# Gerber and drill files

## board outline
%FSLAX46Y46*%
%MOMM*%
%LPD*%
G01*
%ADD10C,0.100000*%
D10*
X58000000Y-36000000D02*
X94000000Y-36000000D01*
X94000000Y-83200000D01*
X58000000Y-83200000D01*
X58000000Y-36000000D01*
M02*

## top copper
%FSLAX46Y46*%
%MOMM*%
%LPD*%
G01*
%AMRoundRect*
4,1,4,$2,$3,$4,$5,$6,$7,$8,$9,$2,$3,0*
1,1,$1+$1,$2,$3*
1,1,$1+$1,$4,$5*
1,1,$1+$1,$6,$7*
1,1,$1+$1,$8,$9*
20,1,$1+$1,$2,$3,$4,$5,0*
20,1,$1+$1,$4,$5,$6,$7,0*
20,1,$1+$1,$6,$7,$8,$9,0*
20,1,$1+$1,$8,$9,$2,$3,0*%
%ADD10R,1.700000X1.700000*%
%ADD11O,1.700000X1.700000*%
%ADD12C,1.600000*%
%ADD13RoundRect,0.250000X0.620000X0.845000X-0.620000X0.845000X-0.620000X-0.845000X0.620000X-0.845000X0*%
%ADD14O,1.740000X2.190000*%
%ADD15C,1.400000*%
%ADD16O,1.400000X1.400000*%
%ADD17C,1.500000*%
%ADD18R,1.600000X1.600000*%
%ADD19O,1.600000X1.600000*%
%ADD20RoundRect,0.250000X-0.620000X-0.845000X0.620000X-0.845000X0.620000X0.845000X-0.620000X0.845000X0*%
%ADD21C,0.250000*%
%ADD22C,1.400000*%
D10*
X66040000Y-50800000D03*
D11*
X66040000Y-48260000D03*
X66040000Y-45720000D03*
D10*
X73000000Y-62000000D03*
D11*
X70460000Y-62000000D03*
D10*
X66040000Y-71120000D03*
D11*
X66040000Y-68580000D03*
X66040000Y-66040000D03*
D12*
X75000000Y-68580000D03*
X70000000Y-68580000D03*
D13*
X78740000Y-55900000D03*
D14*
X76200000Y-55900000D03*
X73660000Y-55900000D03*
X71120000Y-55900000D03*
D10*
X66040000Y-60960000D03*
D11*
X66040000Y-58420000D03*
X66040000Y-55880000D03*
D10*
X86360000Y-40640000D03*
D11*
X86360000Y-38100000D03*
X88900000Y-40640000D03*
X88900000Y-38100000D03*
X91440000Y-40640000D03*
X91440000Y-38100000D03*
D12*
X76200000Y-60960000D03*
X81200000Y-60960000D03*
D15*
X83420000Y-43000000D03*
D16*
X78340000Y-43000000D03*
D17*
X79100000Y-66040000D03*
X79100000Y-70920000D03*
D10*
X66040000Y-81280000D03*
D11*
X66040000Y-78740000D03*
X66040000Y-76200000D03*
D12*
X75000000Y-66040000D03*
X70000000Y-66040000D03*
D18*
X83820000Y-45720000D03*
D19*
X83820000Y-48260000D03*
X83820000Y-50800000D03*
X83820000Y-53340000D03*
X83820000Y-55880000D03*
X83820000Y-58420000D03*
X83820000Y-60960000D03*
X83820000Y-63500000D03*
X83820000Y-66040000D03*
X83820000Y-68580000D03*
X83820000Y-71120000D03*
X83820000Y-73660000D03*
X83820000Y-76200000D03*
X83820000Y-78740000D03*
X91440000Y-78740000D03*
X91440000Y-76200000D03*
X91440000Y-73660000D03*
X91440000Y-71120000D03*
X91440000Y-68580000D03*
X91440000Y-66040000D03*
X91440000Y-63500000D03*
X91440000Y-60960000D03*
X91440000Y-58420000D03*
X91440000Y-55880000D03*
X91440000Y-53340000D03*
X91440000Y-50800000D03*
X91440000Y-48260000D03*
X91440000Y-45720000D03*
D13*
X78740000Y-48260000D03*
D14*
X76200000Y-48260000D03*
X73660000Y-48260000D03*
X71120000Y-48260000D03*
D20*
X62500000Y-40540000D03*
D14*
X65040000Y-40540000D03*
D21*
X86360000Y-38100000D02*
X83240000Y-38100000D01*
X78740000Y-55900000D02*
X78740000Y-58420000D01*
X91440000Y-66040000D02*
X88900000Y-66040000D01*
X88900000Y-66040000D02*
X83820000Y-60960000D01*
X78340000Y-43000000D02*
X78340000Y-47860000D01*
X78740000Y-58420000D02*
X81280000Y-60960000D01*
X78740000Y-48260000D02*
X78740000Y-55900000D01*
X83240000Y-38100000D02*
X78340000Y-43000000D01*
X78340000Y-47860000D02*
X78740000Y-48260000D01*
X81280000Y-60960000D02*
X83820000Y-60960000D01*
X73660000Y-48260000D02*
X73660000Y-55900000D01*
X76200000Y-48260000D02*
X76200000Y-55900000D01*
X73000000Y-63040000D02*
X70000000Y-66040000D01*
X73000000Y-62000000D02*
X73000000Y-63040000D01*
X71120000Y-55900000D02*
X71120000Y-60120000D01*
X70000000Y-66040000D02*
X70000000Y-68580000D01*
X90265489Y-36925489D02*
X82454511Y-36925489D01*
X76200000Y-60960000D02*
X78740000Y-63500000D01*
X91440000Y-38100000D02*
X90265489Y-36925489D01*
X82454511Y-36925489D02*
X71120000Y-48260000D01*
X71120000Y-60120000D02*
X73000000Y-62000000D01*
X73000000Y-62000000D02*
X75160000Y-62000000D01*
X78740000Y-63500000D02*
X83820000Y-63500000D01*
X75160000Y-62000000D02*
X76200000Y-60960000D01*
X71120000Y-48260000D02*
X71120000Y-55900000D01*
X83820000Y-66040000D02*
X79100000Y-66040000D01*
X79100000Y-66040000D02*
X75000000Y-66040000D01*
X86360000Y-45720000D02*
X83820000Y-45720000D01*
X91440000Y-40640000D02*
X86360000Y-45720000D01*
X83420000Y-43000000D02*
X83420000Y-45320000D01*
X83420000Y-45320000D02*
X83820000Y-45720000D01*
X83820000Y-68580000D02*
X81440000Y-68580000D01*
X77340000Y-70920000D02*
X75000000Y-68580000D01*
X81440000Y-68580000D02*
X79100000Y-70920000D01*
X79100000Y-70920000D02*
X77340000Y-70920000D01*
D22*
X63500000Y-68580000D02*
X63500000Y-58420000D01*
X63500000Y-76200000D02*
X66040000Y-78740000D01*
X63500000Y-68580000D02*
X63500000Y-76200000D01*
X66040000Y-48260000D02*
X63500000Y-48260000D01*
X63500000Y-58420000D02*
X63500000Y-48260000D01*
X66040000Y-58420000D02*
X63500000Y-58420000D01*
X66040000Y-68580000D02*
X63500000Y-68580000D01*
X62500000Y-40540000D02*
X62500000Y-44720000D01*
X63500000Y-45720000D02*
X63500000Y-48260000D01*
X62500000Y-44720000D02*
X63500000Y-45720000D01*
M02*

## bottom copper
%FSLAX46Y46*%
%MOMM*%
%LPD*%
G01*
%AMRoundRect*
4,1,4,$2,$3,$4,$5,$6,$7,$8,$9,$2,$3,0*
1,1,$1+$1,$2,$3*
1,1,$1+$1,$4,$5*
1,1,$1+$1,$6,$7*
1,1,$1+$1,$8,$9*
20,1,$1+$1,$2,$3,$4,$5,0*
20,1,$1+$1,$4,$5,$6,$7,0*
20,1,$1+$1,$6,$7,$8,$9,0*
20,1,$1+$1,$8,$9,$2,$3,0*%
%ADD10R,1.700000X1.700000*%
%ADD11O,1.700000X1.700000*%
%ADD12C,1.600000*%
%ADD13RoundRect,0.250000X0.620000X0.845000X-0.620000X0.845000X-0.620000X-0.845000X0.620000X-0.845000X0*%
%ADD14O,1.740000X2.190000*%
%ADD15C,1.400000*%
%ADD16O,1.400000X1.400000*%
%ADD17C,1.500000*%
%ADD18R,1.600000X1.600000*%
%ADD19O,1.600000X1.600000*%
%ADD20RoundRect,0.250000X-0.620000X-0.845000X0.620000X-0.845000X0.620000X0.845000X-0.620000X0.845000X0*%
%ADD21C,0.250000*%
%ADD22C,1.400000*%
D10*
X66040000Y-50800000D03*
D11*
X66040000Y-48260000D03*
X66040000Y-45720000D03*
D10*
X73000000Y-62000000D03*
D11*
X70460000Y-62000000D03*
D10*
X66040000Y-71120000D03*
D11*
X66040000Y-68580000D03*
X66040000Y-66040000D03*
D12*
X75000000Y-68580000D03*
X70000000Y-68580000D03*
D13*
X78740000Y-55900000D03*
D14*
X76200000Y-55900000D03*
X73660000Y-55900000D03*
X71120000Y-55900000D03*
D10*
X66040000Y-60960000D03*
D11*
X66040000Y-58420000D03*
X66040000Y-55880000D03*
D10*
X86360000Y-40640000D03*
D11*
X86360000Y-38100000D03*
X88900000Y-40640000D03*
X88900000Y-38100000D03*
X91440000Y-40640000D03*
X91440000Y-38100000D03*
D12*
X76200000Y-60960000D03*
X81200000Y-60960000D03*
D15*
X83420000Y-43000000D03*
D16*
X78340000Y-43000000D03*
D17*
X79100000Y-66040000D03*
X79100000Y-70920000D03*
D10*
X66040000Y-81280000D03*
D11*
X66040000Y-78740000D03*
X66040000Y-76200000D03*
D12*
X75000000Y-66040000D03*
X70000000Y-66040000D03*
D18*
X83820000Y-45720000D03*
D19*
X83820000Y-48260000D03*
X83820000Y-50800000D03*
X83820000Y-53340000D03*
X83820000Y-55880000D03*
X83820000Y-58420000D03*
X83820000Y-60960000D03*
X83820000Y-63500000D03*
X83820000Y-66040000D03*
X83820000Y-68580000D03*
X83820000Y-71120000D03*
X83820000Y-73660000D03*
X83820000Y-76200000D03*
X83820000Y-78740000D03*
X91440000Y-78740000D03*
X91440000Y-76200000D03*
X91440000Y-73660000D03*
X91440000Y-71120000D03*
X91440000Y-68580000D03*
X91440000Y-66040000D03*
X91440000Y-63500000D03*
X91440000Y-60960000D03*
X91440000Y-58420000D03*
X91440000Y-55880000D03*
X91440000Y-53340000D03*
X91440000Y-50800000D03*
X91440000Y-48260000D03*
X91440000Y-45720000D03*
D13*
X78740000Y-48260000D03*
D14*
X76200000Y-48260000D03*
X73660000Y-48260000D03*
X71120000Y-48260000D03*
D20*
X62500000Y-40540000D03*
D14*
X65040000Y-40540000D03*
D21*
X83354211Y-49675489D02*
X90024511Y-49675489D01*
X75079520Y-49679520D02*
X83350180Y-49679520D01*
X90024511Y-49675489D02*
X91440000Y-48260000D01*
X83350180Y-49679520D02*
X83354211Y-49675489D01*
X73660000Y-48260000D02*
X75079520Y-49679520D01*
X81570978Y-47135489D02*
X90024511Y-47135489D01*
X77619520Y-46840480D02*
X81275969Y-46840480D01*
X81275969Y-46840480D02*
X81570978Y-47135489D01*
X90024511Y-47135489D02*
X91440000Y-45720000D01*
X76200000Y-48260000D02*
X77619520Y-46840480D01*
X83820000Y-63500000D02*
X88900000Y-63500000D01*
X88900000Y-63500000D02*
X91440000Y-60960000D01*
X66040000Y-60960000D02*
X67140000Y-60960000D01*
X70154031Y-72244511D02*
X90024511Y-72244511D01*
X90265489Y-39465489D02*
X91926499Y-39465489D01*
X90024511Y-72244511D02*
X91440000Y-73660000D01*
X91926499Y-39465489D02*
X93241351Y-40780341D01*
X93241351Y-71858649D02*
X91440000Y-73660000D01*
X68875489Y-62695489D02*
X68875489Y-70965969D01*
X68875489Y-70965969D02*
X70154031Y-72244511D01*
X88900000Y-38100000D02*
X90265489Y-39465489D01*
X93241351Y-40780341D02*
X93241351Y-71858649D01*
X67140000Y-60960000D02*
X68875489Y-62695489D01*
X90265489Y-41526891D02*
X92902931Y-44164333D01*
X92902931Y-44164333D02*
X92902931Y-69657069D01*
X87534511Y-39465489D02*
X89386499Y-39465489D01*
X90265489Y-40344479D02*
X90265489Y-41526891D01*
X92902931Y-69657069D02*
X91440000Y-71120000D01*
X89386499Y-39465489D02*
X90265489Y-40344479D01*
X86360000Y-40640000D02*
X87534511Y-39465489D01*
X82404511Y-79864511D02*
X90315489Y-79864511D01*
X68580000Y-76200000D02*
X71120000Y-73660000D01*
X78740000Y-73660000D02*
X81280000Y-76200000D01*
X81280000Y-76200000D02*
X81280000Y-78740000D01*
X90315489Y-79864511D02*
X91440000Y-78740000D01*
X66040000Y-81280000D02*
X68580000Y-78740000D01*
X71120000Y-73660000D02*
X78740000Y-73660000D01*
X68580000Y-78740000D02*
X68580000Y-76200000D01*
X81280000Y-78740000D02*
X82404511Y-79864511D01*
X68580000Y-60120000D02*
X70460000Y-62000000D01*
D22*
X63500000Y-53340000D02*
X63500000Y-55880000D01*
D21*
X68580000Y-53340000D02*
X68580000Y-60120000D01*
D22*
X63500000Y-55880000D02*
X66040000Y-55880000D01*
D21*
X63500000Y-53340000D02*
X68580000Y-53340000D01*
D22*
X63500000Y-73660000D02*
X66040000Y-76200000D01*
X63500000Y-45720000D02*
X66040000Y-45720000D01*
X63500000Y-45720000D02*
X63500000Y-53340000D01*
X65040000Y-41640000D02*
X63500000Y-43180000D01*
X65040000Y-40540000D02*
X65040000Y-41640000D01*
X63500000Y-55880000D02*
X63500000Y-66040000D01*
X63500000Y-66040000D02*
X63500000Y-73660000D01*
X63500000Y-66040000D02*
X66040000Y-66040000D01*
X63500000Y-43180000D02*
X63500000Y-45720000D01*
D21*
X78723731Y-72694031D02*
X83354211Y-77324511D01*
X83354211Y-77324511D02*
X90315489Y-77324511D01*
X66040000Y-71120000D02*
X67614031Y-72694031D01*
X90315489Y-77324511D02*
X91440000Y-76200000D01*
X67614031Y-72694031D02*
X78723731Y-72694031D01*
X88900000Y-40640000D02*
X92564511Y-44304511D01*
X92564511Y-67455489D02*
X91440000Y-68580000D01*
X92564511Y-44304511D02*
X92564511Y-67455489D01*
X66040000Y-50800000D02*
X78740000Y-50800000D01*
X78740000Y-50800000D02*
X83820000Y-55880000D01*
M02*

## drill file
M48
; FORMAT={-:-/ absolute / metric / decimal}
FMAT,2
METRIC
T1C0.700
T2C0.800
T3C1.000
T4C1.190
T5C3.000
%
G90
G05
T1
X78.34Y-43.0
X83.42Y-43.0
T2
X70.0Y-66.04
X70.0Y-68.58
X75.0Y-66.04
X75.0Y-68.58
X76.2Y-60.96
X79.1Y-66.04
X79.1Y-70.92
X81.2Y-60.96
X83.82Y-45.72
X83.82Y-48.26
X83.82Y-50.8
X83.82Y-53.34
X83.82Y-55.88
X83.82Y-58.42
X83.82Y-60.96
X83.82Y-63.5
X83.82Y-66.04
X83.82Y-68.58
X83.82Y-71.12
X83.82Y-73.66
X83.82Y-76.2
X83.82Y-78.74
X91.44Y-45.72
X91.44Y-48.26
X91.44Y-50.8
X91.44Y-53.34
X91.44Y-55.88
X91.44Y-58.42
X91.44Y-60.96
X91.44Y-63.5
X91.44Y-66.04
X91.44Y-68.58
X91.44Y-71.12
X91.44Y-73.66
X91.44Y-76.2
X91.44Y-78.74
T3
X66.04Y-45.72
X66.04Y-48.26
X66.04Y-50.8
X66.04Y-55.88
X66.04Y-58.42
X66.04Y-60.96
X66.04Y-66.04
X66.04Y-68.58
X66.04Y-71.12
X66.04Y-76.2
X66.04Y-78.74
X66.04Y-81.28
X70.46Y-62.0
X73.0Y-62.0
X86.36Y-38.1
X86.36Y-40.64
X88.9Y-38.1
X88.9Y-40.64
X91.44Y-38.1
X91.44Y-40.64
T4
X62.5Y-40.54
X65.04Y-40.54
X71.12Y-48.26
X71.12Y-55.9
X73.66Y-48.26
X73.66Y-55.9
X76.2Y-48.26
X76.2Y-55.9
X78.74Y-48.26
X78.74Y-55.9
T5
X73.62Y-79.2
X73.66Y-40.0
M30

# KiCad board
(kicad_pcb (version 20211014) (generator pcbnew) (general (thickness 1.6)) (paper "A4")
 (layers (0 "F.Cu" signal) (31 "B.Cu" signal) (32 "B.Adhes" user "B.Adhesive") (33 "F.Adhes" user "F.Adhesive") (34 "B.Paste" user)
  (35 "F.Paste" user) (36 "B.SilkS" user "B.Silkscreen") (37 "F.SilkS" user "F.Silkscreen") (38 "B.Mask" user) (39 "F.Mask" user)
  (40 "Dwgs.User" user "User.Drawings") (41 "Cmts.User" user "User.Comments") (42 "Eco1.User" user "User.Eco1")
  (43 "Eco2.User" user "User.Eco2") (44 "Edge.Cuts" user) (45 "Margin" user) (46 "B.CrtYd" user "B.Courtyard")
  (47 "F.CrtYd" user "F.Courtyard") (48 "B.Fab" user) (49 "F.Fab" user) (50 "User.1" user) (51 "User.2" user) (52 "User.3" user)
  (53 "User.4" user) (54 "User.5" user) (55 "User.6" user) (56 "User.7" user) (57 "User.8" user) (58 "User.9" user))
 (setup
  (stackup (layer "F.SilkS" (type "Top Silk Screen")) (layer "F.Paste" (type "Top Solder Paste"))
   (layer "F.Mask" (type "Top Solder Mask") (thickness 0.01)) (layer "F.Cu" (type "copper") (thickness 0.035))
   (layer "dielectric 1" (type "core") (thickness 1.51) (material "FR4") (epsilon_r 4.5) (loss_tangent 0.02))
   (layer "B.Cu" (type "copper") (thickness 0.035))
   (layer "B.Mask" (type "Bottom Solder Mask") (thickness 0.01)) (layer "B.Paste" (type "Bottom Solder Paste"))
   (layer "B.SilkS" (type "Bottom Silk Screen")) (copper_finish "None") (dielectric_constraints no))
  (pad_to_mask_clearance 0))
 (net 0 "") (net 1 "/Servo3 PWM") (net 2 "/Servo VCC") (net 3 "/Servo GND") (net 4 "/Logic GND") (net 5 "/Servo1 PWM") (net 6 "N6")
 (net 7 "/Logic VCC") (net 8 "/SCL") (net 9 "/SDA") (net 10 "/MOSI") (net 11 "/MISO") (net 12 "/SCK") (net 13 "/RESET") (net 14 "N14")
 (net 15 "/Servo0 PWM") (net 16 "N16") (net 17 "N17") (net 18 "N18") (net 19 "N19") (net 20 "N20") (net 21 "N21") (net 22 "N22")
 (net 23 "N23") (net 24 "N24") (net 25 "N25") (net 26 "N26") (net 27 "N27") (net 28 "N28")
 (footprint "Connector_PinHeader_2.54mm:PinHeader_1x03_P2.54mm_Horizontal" (layer "F.Cu") (at 66.04 50.8 180)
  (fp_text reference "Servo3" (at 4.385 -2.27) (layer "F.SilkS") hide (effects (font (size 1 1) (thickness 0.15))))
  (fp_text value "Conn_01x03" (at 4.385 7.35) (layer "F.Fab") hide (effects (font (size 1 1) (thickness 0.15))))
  (pad "1" thru_hole rect (at 0 0 180) (size 1.7 1.7) (drill 1) (layers *.Cu *.Mask) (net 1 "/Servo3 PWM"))
  (pad "2" thru_hole oval (at 0 2.54 180) (size 1.7 1.7) (drill 1) (layers *.Cu *.Mask) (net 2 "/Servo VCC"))
  (pad "3" thru_hole oval (at 0 5.08 180) (size 1.7 1.7) (drill 1) (layers *.Cu *.Mask) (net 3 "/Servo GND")))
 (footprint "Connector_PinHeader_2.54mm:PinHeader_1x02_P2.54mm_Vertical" (layer "F.Cu") (at 73 62 -90)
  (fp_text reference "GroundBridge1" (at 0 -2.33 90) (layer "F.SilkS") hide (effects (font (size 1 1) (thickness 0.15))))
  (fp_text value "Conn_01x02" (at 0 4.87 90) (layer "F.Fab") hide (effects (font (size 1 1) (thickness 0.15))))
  (pad "1" thru_hole rect (at 0 0 270) (size 1.7 1.7) (drill 1) (layers *.Cu *.Mask) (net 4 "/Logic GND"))
  (pad "2" thru_hole oval (at 0 2.54 270) (size 1.7 1.7) (drill 1) (layers *.Cu *.Mask) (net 3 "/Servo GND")))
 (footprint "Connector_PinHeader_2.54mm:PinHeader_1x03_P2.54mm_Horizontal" (layer "F.Cu") (at 66.04 71.12 180)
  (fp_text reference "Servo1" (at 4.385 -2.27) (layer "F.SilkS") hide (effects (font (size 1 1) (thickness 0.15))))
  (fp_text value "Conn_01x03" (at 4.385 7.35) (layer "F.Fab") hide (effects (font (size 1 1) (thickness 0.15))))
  (pad "1" thru_hole rect (at 0 0 180) (size 1.7 1.7) (drill 1) (layers *.Cu *.Mask) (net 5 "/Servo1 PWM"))
  (pad "2" thru_hole oval (at 0 2.54 180) (size 1.7 1.7) (drill 1) (layers *.Cu *.Mask) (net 2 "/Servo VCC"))
  (pad "3" thru_hole oval (at 0 5.08 180) (size 1.7 1.7) (drill 1) (layers *.Cu *.Mask) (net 3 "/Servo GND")))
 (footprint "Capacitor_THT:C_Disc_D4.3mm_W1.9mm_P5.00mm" (layer "F.Cu") (at 75 68.58 180)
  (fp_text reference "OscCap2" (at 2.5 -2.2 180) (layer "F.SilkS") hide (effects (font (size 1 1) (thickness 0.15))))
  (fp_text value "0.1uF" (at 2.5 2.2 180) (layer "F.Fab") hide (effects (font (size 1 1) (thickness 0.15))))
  (pad "1" thru_hole circle (at 0 0 180) (size 1.6 1.6) (drill 0.8) (layers *.Cu *.Mask) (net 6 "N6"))
  (pad "2" thru_hole circle (at 5 0 180) (size 1.6 1.6) (drill 0.8) (layers *.Cu *.Mask) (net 4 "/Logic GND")))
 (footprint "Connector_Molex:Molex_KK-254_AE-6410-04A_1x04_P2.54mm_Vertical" (layer "F.Cu") (at 78.74 55.9 180)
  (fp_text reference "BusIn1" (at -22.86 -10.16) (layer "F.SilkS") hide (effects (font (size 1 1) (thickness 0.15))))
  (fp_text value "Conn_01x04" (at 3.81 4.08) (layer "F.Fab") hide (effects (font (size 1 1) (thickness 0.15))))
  (pad "1" thru_hole roundrect (at 0 0 180) (size 1.74 2.19) (drill 1.19) (layers *.Cu *.Mask) (roundrect_rratio 0.1436781609)
   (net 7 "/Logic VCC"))
  (pad "2" thru_hole oval (at 2.54 0 180) (size 1.74 2.19) (drill 1.19) (layers *.Cu *.Mask) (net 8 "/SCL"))
  (pad "3" thru_hole oval (at 5.08 0 180) (size 1.74 2.19) (drill 1.19) (layers *.Cu *.Mask) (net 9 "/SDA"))
  (pad "4" thru_hole oval (at 7.62 0 180) (size 1.74 2.19) (drill 1.19) (layers *.Cu *.Mask) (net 4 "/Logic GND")))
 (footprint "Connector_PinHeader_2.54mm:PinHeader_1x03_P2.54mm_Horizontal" (layer "F.Cu") (at 66.04 60.96 180)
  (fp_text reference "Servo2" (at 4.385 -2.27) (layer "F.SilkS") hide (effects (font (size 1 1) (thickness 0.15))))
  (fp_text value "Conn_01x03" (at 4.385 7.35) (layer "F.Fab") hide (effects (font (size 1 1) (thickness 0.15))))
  (pad "1" thru_hole rect (at 0 0 180) (size 1.7 1.7) (drill 1) (layers *.Cu *.Mask) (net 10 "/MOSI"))
  (pad "2" thru_hole oval (at 0 2.54 180) (size 1.7 1.7) (drill 1) (layers *.Cu *.Mask) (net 2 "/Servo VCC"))
  (pad "3" thru_hole oval (at 0 5.08 180) (size 1.7 1.7) (drill 1) (layers *.Cu *.Mask) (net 3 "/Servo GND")))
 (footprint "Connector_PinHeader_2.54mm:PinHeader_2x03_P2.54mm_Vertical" (layer "F.Cu") (at 86.36 40.64 90)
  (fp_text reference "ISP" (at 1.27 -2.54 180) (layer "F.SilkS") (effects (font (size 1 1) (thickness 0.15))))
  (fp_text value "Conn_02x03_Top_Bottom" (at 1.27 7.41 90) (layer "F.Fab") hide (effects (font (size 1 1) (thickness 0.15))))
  (pad "1" thru_hole rect (at 0 0 90) (size 1.7 1.7) (drill 1) (layers *.Cu *.Mask) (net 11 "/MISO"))
  (pad "2" thru_hole oval (at 2.54 0 90) (size 1.7 1.7) (drill 1) (layers *.Cu *.Mask) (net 7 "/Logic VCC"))
  (pad "3" thru_hole oval (at 0 2.54 90) (size 1.7 1.7) (drill 1) (layers *.Cu *.Mask) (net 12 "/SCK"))
  (pad "4" thru_hole oval (at 2.54 2.54 90) (size 1.7 1.7) (drill 1) (layers *.Cu *.Mask) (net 10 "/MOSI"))
  (pad "5" thru_hole oval (at 0 5.08 90) (size 1.7 1.7) (drill 1) (layers *.Cu *.Mask) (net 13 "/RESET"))
  (pad "6" thru_hole oval (at 2.54 5.08 90) (size 1.7 1.7) (drill 1) (layers *.Cu *.Mask) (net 4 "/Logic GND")))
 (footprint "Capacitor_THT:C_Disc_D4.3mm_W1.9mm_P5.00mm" (layer "F.Cu") (at 76.2 60.96)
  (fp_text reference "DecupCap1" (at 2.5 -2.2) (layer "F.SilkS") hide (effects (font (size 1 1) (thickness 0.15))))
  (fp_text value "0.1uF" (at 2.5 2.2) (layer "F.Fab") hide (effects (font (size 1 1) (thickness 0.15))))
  (pad "1" thru_hole circle (at 0 0) (size 1.6 1.6) (drill 0.8) (layers *.Cu *.Mask) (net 4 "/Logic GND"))
  (pad "2" thru_hole circle (at 5 0) (size 1.6 1.6) (drill 0.8) (layers *.Cu *.Mask) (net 7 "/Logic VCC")))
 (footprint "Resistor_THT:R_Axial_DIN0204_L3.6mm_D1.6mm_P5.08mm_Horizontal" (layer "F.Cu") (at 83.42 43 180)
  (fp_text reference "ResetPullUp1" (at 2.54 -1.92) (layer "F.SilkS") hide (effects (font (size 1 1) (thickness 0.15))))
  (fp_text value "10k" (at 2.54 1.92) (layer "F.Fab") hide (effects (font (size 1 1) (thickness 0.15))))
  (pad "1" thru_hole circle (at 0 0 180) (size 1.4 1.4) (drill 0.7) (layers *.Cu *.Mask) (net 13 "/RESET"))
  (pad "2" thru_hole oval (at 5.08 0 180) (size 1.4 1.4) (drill 0.7) (layers *.Cu *.Mask) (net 7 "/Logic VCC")))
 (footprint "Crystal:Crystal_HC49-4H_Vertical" (layer "F.Cu") (at 79.1 66.04 -90)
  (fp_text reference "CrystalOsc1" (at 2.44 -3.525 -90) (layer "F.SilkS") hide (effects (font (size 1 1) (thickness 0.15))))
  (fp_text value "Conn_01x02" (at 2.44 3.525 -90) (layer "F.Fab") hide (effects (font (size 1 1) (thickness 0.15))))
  (pad "1" thru_hole circle (at 0 0 270) (size 1.5 1.5) (drill 0.8) (layers *.Cu *.Mask) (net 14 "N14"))
  (pad "2" thru_hole circle (at 4.88 0 270) (size 1.5 1.5) (drill 0.8) (layers *.Cu *.Mask) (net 6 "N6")))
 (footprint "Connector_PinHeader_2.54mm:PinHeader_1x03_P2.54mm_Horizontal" (layer "F.Cu") (at 66.04 81.28 180)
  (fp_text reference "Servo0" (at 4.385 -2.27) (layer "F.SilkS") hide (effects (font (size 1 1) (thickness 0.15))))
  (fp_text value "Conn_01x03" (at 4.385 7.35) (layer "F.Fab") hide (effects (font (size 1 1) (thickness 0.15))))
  (pad "1" thru_hole rect (at 0 0 180) (size 1.7 1.7) (drill 1) (layers *.Cu *.Mask) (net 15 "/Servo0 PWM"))
  (pad "2" thru_hole oval (at 0 2.54 180) (size 1.7 1.7) (drill 1) (layers *.Cu *.Mask) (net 2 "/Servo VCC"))
  (pad "3" thru_hole oval (at 0 5.08 180) (size 1.7 1.7) (drill 1) (layers *.Cu *.Mask) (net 3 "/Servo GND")))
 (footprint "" (layer "F.Cu") (at 73.66 40)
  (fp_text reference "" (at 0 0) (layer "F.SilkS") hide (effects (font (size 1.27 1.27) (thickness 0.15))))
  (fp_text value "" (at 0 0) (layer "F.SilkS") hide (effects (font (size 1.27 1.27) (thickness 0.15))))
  (pad "" np_thru_hole circle (at 0 0) (size 6 6) (drill 3) (layers *.Mask)))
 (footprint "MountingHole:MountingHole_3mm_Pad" (layer "F.Cu") (at 73.62 79.2)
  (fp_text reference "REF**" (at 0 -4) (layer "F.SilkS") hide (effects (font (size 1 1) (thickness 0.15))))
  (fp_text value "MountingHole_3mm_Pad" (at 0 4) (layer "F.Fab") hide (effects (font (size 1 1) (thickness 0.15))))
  (pad "" np_thru_hole circle (at 0 0) (size 6 6) (drill 3) (layers *.Mask)))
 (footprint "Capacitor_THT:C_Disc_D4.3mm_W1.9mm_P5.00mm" (layer "F.Cu") (at 75 66.04 180)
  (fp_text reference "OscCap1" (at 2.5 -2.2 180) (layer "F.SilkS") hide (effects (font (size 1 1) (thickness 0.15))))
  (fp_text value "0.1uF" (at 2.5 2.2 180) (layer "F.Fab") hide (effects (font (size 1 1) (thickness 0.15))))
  (pad "1" thru_hole circle (at 0 0 180) (size 1.6 1.6) (drill 0.8) (layers *.Cu *.Mask) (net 14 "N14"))
  (pad "2" thru_hole circle (at 5 0 180) (size 1.6 1.6) (drill 0.8) (layers *.Cu *.Mask) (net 4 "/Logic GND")))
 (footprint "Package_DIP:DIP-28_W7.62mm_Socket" (layer "F.Cu") (at 83.82 45.72)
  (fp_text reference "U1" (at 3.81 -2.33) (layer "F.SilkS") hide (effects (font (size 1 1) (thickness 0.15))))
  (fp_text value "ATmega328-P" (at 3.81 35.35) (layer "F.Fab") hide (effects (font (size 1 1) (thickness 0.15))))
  (pad "1" thru_hole rect (at 0 0) (size 1.6 1.6) (drill 0.8) (layers *.Cu *.Mask) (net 13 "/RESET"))
  (pad "2" thru_hole oval (at 0 2.54) (size 1.6 1.6) (drill 0.8) (layers *.Cu *.Mask) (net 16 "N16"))
  (pad "3" thru_hole oval (at 0 5.08) (size 1.6 1.6) (drill 0.8) (layers *.Cu *.Mask) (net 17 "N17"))
  (pad "4" thru_hole oval (at 0 7.62) (size 1.6 1.6) (drill 0.8) (layers *.Cu *.Mask) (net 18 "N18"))
  (pad "5" thru_hole oval (at 0 10.16) (size 1.6 1.6) (drill 0.8) (layers *.Cu *.Mask) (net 1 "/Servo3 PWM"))
  (pad "6" thru_hole oval (at 0 12.7) (size 1.6 1.6) (drill 0.8) (layers *.Cu *.Mask) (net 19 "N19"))
  (pad "7" thru_hole oval (at 0 15.24) (size 1.6 1.6) (drill 0.8) (layers *.Cu *.Mask) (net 7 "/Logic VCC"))
  (pad "8" thru_hole oval (at 0 17.78) (size 1.6 1.6) (drill 0.8) (layers *.Cu *.Mask) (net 4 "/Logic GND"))
  (pad "9" thru_hole oval (at 0 20.32) (size 1.6 1.6) (drill 0.8) (layers *.Cu *.Mask) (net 14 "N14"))
  (pad "10" thru_hole oval (at 0 22.86) (size 1.6 1.6) (drill 0.8) (layers *.Cu *.Mask) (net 6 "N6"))
  (pad "11" thru_hole oval (at 0 25.4) (size 1.6 1.6) (drill 0.8) (layers *.Cu *.Mask) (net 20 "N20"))
  (pad "12" thru_hole oval (at 0 27.94) (size 1.6 1.6) (drill 0.8) (layers *.Cu *.Mask) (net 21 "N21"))
  (pad "13" thru_hole oval (at 0 30.48) (size 1.6 1.6) (drill 0.8) (layers *.Cu *.Mask) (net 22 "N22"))
  (pad "14" thru_hole oval (at 0 33.02) (size 1.6 1.6) (drill 0.8) (layers *.Cu *.Mask) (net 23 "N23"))
  (pad "15" thru_hole oval (at 7.62 33.02) (size 1.6 1.6) (drill 0.8) (layers *.Cu *.Mask) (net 15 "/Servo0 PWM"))
  (pad "16" thru_hole oval (at 7.62 30.48) (size 1.6 1.6) (drill 0.8) (layers *.Cu *.Mask) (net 5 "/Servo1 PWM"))
  (pad "17" thru_hole oval (at 7.62 27.94) (size 1.6 1.6) (drill 0.8) (layers *.Cu *.Mask) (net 10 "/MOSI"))
  (pad "18" thru_hole oval (at 7.62 25.4) (size 1.6 1.6) (drill 0.8) (layers *.Cu *.Mask) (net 11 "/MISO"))
  (pad "19" thru_hole oval (at 7.62 22.86) (size 1.6 1.6) (drill 0.8) (layers *.Cu *.Mask) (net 12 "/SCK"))
  (pad "20" thru_hole oval (at 7.62 20.32) (size 1.6 1.6) (drill 0.8) (layers *.Cu *.Mask) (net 7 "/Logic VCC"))
  (pad "21" thru_hole oval (at 7.62 17.78) (size 1.6 1.6) (drill 0.8) (layers *.Cu *.Mask) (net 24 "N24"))
  (pad "22" thru_hole oval (at 7.62 15.24) (size 1.6 1.6) (drill 0.8) (layers *.Cu *.Mask) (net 4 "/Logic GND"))
  (pad "23" thru_hole oval (at 7.62 12.7) (size 1.6 1.6) (drill 0.8) (layers *.Cu *.Mask) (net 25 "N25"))
  (pad "24" thru_hole oval (at 7.62 10.16) (size 1.6 1.6) (drill 0.8) (layers *.Cu *.Mask) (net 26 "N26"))
  (pad "25" thru_hole oval (at 7.62 7.62) (size 1.6 1.6) (drill 0.8) (layers *.Cu *.Mask) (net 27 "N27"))
  (pad "26" thru_hole oval (at 7.62 5.08) (size 1.6 1.6) (drill 0.8) (layers *.Cu *.Mask) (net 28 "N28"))
  (pad "27" thru_hole oval (at 7.62 2.54) (size 1.6 1.6) (drill 0.8) (layers *.Cu *.Mask) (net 9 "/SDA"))
  (pad "28" thru_hole oval (at 7.62 0) (size 1.6 1.6) (drill 0.8) (layers *.Cu *.Mask) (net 8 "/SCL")))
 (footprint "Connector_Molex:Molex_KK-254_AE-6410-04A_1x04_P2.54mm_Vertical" (layer "F.Cu") (at 78.74 48.26 180)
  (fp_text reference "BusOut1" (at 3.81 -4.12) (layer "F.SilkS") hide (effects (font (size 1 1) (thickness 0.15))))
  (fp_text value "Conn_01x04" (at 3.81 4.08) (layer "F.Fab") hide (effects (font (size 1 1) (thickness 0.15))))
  (pad "1" thru_hole roundrect (at 0 0 180) (size 1.74 2.19) (drill 1.19) (layers *.Cu *.Mask) (roundrect_rratio 0.1436781609)
   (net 7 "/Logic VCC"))
  (pad "2" thru_hole oval (at 2.54 0 180) (size 1.74 2.19) (drill 1.19) (layers *.Cu *.Mask) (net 8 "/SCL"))
  (pad "3" thru_hole oval (at 5.08 0 180) (size 1.74 2.19) (drill 1.19) (layers *.Cu *.Mask) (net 9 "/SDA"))
  (pad "4" thru_hole oval (at 7.62 0 180) (size 1.74 2.19) (drill 1.19) (layers *.Cu *.Mask) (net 4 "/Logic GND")))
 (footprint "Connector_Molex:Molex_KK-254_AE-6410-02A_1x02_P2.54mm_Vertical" (layer "F.Cu") (at 62.5 40.54)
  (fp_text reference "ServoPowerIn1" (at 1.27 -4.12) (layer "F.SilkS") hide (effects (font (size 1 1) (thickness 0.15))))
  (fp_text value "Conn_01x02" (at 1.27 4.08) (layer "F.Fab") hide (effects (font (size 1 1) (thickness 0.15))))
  (pad "1" thru_hole roundrect (at 0 0) (size 1.74 2.19) (drill 1.19) (layers *.Cu *.Mask) (roundrect_rratio 0.1436781609)
   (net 2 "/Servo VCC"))
  (pad "2" thru_hole oval (at 2.54 0) (size 1.74 2.19) (drill 1.19) (layers *.Cu *.Mask) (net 3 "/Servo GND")))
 (gr_rect (start 58 36) (end 94 83.2) (layer "Edge.Cuts") (width 0.1) (fill none))
 (segment (start 86.36 38.1) (end 83.24 38.1) (width 0.25) (layer "F.Cu") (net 7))
 (segment (start 78.74 55.9) (end 78.74 58.42) (width 0.25) (layer "F.Cu") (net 7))
 (segment (start 91.44 66.04) (end 88.9 66.04) (width 0.25) (layer "F.Cu") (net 7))
 (segment (start 88.9 66.04) (end 83.82 60.96) (width 0.25) (layer "F.Cu") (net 7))
 (segment (start 78.34 43) (end 78.34 47.86) (width 0.25) (layer "F.Cu") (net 7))
 (segment (start 78.74 58.42) (end 81.28 60.96) (width 0.25) (layer "F.Cu") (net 7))
 (segment (start 78.74 48.26) (end 78.74 55.9) (width 0.25) (layer "F.Cu") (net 7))
 (segment (start 83.24 38.1) (end 78.34 43) (width 0.25) (layer "F.Cu") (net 7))
 (segment (start 78.34 47.86) (end 78.74 48.26) (width 0.25) (layer "F.Cu") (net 7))
 (segment (start 81.28 60.96) (end 83.82 60.96) (width 0.25) (layer "F.Cu") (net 7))
 (segment (start 73.66 48.26) (end 73.66 55.9) (width 0.25) (layer "F.Cu") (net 9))
 (segment (start 83.354211 49.675489) (end 90.024511 49.675489) (width 0.25) (layer "B.Cu") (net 9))
 (segment (start 75.07952 49.67952) (end 83.35018 49.67952) (width 0.25) (layer "B.Cu") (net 9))
 (segment (start 90.024511 49.675489) (end 91.44 48.26) (width 0.25) (layer "B.Cu") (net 9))
 (segment (start 83.35018 49.67952) (end 83.354211 49.675489) (width 0.25) (layer "B.Cu") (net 9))
 (segment (start 73.66 48.26) (end 75.07952 49.67952) (width 0.25) (layer "B.Cu") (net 9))
 (segment (start 76.2 48.26) (end 76.2 55.9) (width 0.25) (layer "F.Cu") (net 8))
 (segment (start 81.570978 47.135489) (end 90.024511 47.135489) (width 0.25) (layer "B.Cu") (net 8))
 (segment (start 77.61952 46.84048) (end 81.275969 46.84048) (width 0.25) (layer "B.Cu") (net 8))
 (segment (start 81.275969 46.84048) (end 81.570978 47.135489) (width 0.25) (layer "B.Cu") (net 8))
 (segment (start 90.024511 47.135489) (end 91.44 45.72) (width 0.25) (layer "B.Cu") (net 8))
 (segment (start 76.2 48.26) (end 77.61952 46.84048) (width 0.25) (layer "B.Cu") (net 8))
 (segment (start 73 63.04) (end 70 66.04) (width 0.25) (layer "F.Cu") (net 4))
 (segment (start 73 62) (end 73 63.04) (width 0.25) (layer "F.Cu") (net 4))
 (segment (start 71.12 55.9) (end 71.12 60.12) (width 0.25) (layer "F.Cu") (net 4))
 (segment (start 70 66.04) (end 70 68.58) (width 0.25) (layer "F.Cu") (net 4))
 (segment (start 90.265489 36.925489) (end 82.454511 36.925489) (width 0.25) (layer "F.Cu") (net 4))
 (segment (start 76.2 60.96) (end 78.74 63.5) (width 0.25) (layer "F.Cu") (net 4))
 (segment (start 91.44 38.1) (end 90.265489 36.925489) (width 0.25) (layer "F.Cu") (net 4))
 (segment (start 82.454511 36.925489) (end 71.12 48.26) (width 0.25) (layer "F.Cu") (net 4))
 (segment (start 71.12 60.12) (end 73 62) (width 0.25) (layer "F.Cu") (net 4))
 (segment (start 73 62) (end 75.16 62) (width 0.25) (layer "F.Cu") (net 4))
 (segment (start 78.74 63.5) (end 83.82 63.5) (width 0.25) (layer "F.Cu") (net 4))
 (segment (start 75.16 62) (end 76.2 60.96) (width 0.25) (layer "F.Cu") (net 4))
 (segment (start 71.12 48.26) (end 71.12 55.9) (width 0.25) (layer "F.Cu") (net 4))
 (segment (start 83.82 63.5) (end 88.9 63.5) (width 0.25) (layer "B.Cu") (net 4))
 (segment (start 88.9 63.5) (end 91.44 60.96) (width 0.25) (layer "B.Cu") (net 4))
 (segment (start 83.82 66.04) (end 79.1 66.04) (width 0.25) (layer "F.Cu") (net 14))
 (segment (start 79.1 66.04) (end 75 66.04) (width 0.25) (layer "F.Cu") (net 14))
 (segment (start 86.36 45.72) (end 83.82 45.72) (width 0.25) (layer "F.Cu") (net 13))
 (segment (start 91.44 40.64) (end 86.36 45.72) (width 0.25) (layer "F.Cu") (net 13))
 (segment (start 83.42 43) (end 83.42 45.32) (width 0.25) (layer "F.Cu") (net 13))
 (segment (start 83.42 45.32) (end 83.82 45.72) (width 0.25) (layer "F.Cu") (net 13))
 (segment (start 66.04 60.96) (end 67.14 60.96) (width 0.25) (layer "B.Cu") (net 10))
 (segment (start 70.154031 72.244511) (end 90.024511 72.244511) (width 0.25) (layer "B.Cu") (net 10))
 (segment (start 90.265489 39.465489) (end 91.926499 39.465489) (width 0.25) (layer "B.Cu") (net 10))
 (segment (start 90.024511 72.244511) (end 91.44 73.66) (width 0.25) (layer "B.Cu") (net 10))
 (segment (start 91.926499 39.465489) (end 93.241351 40.780341) (width 0.25) (layer "B.Cu") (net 10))
 (segment (start 93.241351 71.858649) (end 91.44 73.66) (width 0.25) (layer "B.Cu") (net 10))
 (segment (start 68.875489 62.695489) (end 68.875489 70.965969) (width 0.25) (layer "B.Cu") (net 10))
 (segment (start 68.875489 70.965969) (end 70.154031 72.244511) (width 0.25) (layer "B.Cu") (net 10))
 (segment (start 88.9 38.1) (end 90.265489 39.465489) (width 0.25) (layer "B.Cu") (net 10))
 (segment (start 93.241351 40.780341) (end 93.241351 71.858649) (width 0.25) (layer "B.Cu") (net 10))
 (segment (start 67.14 60.96) (end 68.875489 62.695489) (width 0.25) (layer "B.Cu") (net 10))
 (segment (start 90.265489 41.526891) (end 92.902931 44.164333) (width 0.25) (layer "B.Cu") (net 11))
 (segment (start 92.902931 44.164333) (end 92.902931 69.657069) (width 0.25) (layer "B.Cu") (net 11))
 (segment (start 87.534511 39.465489) (end 89.386499 39.465489) (width 0.25) (layer "B.Cu") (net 11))
 (segment (start 90.265489 40.344479) (end 90.265489 41.526891) (width 0.25) (layer "B.Cu") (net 11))
 (segment (start 92.902931 69.657069) (end 91.44 71.12) (width 0.25) (layer "B.Cu") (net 11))
 (segment (start 89.386499 39.465489) (end 90.265489 40.344479) (width 0.25) (layer "B.Cu") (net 11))
 (segment (start 86.36 40.64) (end 87.534511 39.465489) (width 0.25) (layer "B.Cu") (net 11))
 (segment (start 83.82 68.58) (end 81.44 68.58) (width 0.25) (layer "F.Cu") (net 6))
 (segment (start 77.34 70.92) (end 75 68.58) (width 0.25) (layer "F.Cu") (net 6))
 (segment (start 81.44 68.58) (end 79.1 70.92) (width 0.25) (layer "F.Cu") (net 6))
 (segment (start 79.1 70.92) (end 77.34 70.92) (width 0.25) (layer "F.Cu") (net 6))
 (segment (start 82.404511 79.864511) (end 90.315489 79.864511) (width 0.25) (layer "B.Cu") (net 15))
 (segment (start 68.58 76.2) (end 71.12 73.66) (width 0.25) (layer "B.Cu") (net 15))
 (segment (start 78.74 73.66) (end 81.28 76.2) (width 0.25) (layer "B.Cu") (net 15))
 (segment (start 81.28 76.2) (end 81.28 78.74) (width 0.25) (layer "B.Cu") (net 15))
 (segment (start 90.315489 79.864511) (end 91.44 78.74) (width 0.25) (layer "B.Cu") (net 15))
 (segment (start 66.04 81.28) (end 68.58 78.74) (width 0.25) (layer "B.Cu") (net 15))
 (segment (start 71.12 73.66) (end 78.74 73.66) (width 0.25) (layer "B.Cu") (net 15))
 (segment (start 68.58 78.74) (end 68.58 76.2) (width 0.25) (layer "B.Cu") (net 15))
 (segment (start 81.28 78.74) (end 82.404511 79.864511) (width 0.25) (layer "B.Cu") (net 15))
 (segment (start 63.5 68.58) (end 63.5 58.42) (width 1.4) (layer "F.Cu") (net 2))
 (segment (start 63.5 76.2) (end 66.04 78.74) (width 1.4) (layer "F.Cu") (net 2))
 (segment (start 63.5 68.58) (end 63.5 76.2) (width 1.4) (layer "F.Cu") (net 2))
 (segment (start 66.04 48.26) (end 63.5 48.26) (width 1.4) (layer "F.Cu") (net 2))
 (segment (start 63.5 58.42) (end 63.5 48.26) (width 1.4) (layer "F.Cu") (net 2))
 (segment (start 66.04 58.42) (end 63.5 58.42) (width 1.4) (layer "F.Cu") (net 2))
 (segment (start 66.04 68.58) (end 63.5 68.58) (width 1.4) (layer "F.Cu") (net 2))
 (segment (start 62.5 40.54) (end 62.5 44.72) (width 1.4) (layer "F.Cu") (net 2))
 (segment (start 63.5 45.72) (end 63.5 48.26) (width 1.4) (layer "F.Cu") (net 2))
 (segment (start 62.5 44.72) (end 63.5 45.72) (width 1.4) (layer "F.Cu") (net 2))
 (segment (start 68.58 60.12) (end 70.46 62) (width 0.25) (layer "B.Cu") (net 3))
 (segment (start 63.5 53.34) (end 63.5 55.88) (width 1.4) (layer "B.Cu") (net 3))
 (segment (start 68.58 53.34) (end 68.58 60.12) (width 0.25) (layer "B.Cu") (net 3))
 (segment (start 63.5 55.88) (end 66.04 55.88) (width 1.4) (layer "B.Cu") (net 3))
 (segment (start 63.5 53.34) (end 68.58 53.34) (width 0.25) (layer "B.Cu") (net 3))
 (segment (start 63.5 73.66) (end 66.04 76.2) (width 1.4) (layer "B.Cu") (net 3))
 (segment (start 63.5 45.72) (end 66.04 45.72) (width 1.4) (layer "B.Cu") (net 3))
 (segment (start 63.5 45.72) (end 63.5 53.34) (width 1.4) (layer "B.Cu") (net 3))
 (segment (start 65.04 41.64) (end 63.5 43.18) (width 1.4) (layer "B.Cu") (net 3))
 (segment (start 65.04 40.54) (end 65.04 41.64) (width 1.4) (layer "B.Cu") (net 3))
 (segment (start 63.5 55.88) (end 63.5 66.04) (width 1.4) (layer "B.Cu") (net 3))
 (segment (start 63.5 66.04) (end 63.5 73.66) (width 1.4) (layer "B.Cu") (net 3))
 (segment (start 63.5 66.04) (end 66.04 66.04) (width 1.4) (layer "B.Cu") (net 3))
 (segment (start 63.5 43.18) (end 63.5 45.72) (width 1.4) (layer "B.Cu") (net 3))
 (segment (start 78.723731 72.694031) (end 83.354211 77.324511) (width 0.25) (layer "B.Cu") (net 5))
 (segment (start 83.354211 77.324511) (end 90.315489 77.324511) (width 0.25) (layer "B.Cu") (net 5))
 (segment (start 66.04 71.12) (end 67.614031 72.694031) (width 0.25) (layer "B.Cu") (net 5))
 (segment (start 90.315489 77.324511) (end 91.44 76.2) (width 0.25) (layer "B.Cu") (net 5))
 (segment (start 67.614031 72.694031) (end 78.723731 72.694031) (width 0.25) (layer "B.Cu") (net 5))
 (segment (start 88.9 40.64) (end 92.564511 44.304511) (width 0.25) (layer "B.Cu") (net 12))
 (segment (start 92.564511 67.455489) (end 91.44 68.58) (width 0.25) (layer "B.Cu") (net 12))
 (segment (start 92.564511 44.304511) (end 92.564511 67.455489) (width 0.25) (layer "B.Cu") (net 12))
 (segment (start 66.04 50.8) (end 78.74 50.8) (width 0.25) (layer "B.Cu") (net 1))
 (segment (start 78.74 50.8) (end 83.82 55.88) (width 0.25) (layer "B.Cu") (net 1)))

